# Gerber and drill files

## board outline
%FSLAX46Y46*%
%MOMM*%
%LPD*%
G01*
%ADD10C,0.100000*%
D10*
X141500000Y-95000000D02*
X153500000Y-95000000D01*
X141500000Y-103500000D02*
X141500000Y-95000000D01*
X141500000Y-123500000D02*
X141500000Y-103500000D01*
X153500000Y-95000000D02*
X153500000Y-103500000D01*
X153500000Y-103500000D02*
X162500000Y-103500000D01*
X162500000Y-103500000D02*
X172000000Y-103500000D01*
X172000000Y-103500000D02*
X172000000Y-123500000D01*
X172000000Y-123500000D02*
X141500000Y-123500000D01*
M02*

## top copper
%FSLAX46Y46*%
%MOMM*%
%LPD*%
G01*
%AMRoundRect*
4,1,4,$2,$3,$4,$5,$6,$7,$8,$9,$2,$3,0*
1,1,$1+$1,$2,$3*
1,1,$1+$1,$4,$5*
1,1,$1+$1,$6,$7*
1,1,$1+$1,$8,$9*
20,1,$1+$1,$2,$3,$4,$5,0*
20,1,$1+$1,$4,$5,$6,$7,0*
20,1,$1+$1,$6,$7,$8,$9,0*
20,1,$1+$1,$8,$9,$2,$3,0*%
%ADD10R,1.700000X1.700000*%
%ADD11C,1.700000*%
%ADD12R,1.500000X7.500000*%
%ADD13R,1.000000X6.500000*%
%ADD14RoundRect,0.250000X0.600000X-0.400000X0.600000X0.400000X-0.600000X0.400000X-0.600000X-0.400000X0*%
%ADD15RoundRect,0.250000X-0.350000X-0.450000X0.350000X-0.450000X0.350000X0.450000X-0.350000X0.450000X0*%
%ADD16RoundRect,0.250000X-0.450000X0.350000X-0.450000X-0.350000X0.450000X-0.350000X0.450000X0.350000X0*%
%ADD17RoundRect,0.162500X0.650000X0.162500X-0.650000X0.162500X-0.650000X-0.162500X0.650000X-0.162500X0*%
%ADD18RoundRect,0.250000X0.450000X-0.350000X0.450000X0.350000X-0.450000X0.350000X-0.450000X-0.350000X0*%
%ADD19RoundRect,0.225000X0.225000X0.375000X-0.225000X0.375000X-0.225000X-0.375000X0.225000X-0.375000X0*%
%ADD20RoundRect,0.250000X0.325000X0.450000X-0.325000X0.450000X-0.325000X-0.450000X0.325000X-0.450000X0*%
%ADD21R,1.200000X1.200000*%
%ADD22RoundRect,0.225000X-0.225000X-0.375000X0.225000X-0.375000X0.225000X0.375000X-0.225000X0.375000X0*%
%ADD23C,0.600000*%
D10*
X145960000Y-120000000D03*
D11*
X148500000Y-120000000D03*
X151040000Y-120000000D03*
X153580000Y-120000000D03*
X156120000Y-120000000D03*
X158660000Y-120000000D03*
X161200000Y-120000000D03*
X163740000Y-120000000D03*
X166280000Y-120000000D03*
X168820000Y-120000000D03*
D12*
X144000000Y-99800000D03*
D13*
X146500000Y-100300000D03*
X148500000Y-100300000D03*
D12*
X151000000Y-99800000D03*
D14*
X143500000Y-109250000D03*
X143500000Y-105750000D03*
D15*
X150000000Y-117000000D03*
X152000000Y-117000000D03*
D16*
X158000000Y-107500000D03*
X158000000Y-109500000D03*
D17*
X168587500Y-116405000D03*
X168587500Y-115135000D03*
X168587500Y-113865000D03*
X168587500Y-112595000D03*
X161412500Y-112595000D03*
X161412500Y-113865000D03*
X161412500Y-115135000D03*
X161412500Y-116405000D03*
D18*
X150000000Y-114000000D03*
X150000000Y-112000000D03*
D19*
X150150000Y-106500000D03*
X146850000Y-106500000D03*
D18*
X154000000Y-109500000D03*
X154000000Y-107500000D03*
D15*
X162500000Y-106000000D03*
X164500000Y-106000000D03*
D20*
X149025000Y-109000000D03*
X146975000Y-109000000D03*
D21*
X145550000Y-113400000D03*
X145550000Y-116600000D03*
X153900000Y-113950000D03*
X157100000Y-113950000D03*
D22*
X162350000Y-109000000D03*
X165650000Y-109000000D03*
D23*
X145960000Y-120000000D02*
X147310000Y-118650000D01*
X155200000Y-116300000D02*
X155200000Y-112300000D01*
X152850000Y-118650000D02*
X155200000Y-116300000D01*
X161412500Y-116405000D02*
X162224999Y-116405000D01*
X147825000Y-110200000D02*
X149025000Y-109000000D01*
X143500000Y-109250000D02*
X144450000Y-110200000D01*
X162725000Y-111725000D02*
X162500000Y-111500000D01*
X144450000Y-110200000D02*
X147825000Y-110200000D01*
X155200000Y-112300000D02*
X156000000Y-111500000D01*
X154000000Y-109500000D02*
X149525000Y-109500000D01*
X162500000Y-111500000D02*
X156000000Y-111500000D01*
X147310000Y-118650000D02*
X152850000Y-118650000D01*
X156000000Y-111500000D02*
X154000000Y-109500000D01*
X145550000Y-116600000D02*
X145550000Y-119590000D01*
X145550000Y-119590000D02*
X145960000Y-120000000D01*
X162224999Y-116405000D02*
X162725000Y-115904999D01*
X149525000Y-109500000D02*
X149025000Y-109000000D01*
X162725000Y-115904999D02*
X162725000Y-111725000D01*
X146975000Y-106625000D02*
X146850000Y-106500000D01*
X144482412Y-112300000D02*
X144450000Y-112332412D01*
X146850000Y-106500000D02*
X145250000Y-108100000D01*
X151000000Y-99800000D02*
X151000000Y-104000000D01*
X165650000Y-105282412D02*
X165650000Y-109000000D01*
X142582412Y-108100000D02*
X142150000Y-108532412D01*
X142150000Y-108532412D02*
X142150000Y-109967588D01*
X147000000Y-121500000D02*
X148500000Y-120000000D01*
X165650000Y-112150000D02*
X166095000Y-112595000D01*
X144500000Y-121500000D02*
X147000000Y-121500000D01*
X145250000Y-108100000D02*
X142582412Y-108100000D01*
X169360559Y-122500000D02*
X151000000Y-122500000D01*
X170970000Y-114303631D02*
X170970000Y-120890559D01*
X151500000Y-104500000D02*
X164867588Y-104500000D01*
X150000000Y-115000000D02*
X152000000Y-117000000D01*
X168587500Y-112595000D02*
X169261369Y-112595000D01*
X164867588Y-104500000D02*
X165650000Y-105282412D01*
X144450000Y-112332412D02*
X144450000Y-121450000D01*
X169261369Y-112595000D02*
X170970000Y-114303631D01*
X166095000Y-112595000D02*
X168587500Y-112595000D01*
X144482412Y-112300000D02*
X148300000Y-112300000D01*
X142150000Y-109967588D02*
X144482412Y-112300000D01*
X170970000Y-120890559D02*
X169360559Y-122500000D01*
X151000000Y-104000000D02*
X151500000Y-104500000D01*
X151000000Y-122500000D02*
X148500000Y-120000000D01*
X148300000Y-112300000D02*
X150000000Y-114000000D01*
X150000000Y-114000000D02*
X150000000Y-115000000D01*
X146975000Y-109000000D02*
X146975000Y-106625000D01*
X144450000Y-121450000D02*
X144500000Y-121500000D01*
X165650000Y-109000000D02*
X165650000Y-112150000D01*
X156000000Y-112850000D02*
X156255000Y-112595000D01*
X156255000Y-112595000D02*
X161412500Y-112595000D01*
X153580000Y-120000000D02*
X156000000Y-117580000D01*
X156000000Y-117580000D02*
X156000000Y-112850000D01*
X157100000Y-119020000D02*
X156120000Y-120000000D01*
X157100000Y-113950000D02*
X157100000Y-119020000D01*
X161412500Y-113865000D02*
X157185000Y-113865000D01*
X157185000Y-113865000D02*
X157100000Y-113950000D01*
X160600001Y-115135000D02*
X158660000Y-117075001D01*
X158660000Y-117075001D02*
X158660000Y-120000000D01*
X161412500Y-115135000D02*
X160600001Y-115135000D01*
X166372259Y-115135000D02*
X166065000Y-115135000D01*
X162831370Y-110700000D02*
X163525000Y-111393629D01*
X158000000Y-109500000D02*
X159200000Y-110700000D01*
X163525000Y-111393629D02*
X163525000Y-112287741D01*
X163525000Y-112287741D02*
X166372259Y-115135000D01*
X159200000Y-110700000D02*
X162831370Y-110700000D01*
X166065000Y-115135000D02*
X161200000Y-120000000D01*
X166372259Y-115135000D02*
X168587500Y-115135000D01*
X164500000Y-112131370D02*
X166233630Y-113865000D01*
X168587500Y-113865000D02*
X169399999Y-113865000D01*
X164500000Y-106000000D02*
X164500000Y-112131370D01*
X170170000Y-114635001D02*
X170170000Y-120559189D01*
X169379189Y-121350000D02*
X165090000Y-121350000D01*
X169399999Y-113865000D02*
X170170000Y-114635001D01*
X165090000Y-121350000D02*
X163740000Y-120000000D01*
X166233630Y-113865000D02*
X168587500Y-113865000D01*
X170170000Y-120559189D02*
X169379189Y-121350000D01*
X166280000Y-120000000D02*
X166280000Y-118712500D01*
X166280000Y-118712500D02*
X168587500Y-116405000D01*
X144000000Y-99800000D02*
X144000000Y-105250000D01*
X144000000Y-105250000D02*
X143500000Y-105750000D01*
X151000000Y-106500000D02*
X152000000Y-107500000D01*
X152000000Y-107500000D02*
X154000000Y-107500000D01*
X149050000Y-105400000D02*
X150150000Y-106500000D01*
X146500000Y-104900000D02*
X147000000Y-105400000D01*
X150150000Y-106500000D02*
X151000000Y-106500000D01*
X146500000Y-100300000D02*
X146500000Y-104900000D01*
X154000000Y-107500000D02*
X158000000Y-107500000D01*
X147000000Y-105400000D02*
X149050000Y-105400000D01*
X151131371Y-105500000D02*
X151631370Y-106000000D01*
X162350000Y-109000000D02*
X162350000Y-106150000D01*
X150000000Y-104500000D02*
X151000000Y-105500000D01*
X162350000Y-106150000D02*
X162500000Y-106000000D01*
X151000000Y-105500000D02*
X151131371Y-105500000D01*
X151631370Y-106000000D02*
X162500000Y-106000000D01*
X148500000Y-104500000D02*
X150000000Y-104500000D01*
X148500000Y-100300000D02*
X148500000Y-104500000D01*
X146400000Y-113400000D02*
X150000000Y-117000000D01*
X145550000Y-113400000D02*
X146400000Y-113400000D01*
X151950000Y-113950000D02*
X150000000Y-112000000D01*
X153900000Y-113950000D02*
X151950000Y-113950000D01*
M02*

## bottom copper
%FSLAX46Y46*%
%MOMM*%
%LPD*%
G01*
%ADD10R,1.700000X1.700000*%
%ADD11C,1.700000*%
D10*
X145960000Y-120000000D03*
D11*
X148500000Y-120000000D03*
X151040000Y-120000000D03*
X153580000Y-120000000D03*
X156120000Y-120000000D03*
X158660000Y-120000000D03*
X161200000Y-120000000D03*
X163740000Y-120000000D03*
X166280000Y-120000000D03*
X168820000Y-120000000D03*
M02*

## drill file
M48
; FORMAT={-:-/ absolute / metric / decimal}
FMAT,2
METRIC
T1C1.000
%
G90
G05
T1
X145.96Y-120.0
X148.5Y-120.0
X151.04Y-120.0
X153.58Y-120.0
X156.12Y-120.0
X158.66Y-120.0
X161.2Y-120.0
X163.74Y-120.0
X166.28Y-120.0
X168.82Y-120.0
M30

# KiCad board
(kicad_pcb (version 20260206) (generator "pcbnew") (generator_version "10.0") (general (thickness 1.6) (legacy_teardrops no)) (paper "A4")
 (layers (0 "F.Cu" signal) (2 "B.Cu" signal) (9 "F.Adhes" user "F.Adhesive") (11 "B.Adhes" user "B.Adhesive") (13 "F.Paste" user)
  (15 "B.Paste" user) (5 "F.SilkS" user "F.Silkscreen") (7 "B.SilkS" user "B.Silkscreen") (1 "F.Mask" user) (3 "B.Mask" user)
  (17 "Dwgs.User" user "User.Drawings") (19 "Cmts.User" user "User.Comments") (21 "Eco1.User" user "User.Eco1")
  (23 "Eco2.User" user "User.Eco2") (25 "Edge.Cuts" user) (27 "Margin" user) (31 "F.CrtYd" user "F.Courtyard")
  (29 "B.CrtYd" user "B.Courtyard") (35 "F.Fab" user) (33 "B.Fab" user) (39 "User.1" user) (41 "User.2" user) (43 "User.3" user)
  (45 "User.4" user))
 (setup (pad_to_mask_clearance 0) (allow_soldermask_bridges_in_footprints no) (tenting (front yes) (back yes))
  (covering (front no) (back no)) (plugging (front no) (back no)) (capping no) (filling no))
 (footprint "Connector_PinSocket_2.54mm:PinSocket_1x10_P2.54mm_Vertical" (layer "F.Cu") (at 145.96 120 90)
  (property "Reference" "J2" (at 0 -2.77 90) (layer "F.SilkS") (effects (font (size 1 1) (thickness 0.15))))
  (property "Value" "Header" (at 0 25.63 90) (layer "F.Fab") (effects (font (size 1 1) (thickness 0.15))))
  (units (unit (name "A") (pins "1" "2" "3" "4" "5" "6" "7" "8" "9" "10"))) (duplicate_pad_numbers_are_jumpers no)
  (pad "1" thru_hole rect (at 0 0 90) (size 1.7 1.7) (drill 1) (layers "*.Cu" "*.Mask") (remove_unused_layers no) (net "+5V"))
  (pad "2" thru_hole circle (at 0 2.54 90) (size 1.7 1.7) (drill 1) (layers "*.Cu" "*.Mask") (remove_unused_layers no) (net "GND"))
  (pad "3" thru_hole circle (at 0 5.08 90) (size 1.7 1.7) (drill 1) (layers "*.Cu" "*.Mask") (remove_unused_layers no)
   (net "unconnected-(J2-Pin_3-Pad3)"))
  (pad "4" thru_hole circle (at 0 7.62 90) (size 1.7 1.7) (drill 1) (layers "*.Cu" "*.Mask") (remove_unused_layers no)
   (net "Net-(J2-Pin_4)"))
  (pad "5" thru_hole circle (at 0 10.16 90) (size 1.7 1.7) (drill 1) (layers "*.Cu" "*.Mask") (remove_unused_layers no) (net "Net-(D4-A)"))
  (pad "6" thru_hole circle (at 0 12.7 90) (size 1.7 1.7) (drill 1) (layers "*.Cu" "*.Mask") (remove_unused_layers no)
   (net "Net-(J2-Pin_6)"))
  (pad "7" thru_hole circle (at 0 15.24 90) (size 1.7 1.7) (drill 1) (layers "*.Cu" "*.Mask") (remove_unused_layers no)
   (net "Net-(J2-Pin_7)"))
  (pad "8" thru_hole circle (at 0 17.78 90) (size 1.7 1.7) (drill 1) (layers "*.Cu" "*.Mask") (remove_unused_layers no)
   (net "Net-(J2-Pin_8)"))
  (pad "9" thru_hole circle (at 0 20.32 90) (size 1.7 1.7) (drill 1) (layers "*.Cu" "*.Mask") (remove_unused_layers no)
   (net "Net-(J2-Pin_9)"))
  (pad "10" thru_hole circle (at 0 22.86 90) (size 1.7 1.7) (drill 1) (layers "*.Cu" "*.Mask") (remove_unused_layers no)
   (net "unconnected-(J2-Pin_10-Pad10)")))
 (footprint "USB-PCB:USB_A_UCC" (layer "F.Cu") (at 147.5 100 -90)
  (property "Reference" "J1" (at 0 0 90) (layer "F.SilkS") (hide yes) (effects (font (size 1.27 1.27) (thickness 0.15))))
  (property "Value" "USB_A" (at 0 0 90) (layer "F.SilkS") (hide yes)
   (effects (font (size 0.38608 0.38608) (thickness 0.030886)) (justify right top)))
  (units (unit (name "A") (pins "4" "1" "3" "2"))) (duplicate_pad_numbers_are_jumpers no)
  (pad "1" smd rect (at -0.2 3.5 270) (size 7.5 1.5) (layers "F.Cu" "F.Mask" "F.Paste") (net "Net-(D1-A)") (solder_mask_margin 0.1016))
  (pad "2" smd rect (at 0.3 1 270) (size 6.5 1) (layers "F.Cu" "F.Mask" "F.Paste") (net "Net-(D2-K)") (solder_mask_margin 0.1016))
  (pad "3" smd rect (at 0.3 -1 270) (size 6.5 1) (layers "F.Cu" "F.Mask" "F.Paste") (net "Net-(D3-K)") (solder_mask_margin 0.1016))
  (pad "4" smd rect (at -0.2 -3.5 270) (size 7.5 1.5) (layers "F.Cu" "F.Mask" "F.Paste") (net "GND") (solder_mask_margin 0.1016)))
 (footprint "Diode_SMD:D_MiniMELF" (layer "F.Cu") (at 143.5 107.5 90)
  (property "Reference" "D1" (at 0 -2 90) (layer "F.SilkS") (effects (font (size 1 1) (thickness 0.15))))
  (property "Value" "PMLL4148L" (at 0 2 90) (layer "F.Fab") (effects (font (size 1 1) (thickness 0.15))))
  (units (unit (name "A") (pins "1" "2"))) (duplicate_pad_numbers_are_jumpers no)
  (pad "1" smd roundrect (at -1.75 0 90) (size 1.3 1.7) (layers "F.Cu" "F.Mask" "F.Paste") (roundrect_rratio 0.1923076923) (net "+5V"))
  (pad "2" smd roundrect (at 1.75 0 90) (size 1.3 1.7) (layers "F.Cu" "F.Mask" "F.Paste") (roundrect_rratio 0.1923076923) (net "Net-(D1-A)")))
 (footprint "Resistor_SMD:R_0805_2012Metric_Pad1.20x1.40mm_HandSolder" (layer "F.Cu") (at 151 117)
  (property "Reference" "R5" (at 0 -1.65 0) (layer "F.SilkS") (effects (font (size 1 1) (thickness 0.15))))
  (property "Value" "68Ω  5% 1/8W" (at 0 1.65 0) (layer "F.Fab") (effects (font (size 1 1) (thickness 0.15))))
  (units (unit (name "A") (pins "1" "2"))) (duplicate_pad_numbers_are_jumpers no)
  (pad "1" smd roundrect (at -1 0) (size 1.2 1.4) (layers "F.Cu" "F.Mask" "F.Paste") (roundrect_rratio 0.208333) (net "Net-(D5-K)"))
  (pad "2" smd roundrect (at 1 0) (size 1.2 1.4) (layers "F.Cu" "F.Mask" "F.Paste") (roundrect_rratio 0.208333) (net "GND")))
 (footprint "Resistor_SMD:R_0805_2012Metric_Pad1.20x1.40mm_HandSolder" (layer "F.Cu") (at 158 108.5 -90)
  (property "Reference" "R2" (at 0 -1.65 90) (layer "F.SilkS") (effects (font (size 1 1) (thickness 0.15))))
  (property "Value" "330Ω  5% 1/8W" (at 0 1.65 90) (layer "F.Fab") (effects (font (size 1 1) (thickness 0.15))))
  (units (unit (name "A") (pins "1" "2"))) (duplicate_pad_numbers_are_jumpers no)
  (pad "1" smd roundrect (at -1 0 270) (size 1.2 1.4) (layers "F.Cu" "F.Mask" "F.Paste") (roundrect_rratio 0.208333) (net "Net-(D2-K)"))
  (pad "2" smd roundrect (at 1 0 270) (size 1.2 1.4) (layers "F.Cu" "F.Mask" "F.Paste") (roundrect_rratio 0.208333) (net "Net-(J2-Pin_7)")))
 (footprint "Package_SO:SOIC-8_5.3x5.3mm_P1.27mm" (layer "F.Cu") (at 165 114.5 180)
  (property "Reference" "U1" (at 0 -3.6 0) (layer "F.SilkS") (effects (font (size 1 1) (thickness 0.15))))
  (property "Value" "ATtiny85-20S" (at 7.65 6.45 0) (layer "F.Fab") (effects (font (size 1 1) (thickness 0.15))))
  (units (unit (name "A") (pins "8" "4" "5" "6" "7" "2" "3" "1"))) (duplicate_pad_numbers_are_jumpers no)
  (pad "1" smd roundrect (at -3.5875 -1.905 180) (size 1.625 0.65) (layers "F.Cu" "F.Mask" "F.Paste") (roundrect_rratio 0.25)
   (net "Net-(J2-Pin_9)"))
  (pad "2" smd roundrect (at -3.5875 -0.635 180) (size 1.625 0.65) (layers "F.Cu" "F.Mask" "F.Paste") (roundrect_rratio 0.25)
   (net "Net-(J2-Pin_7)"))
  (pad "3" smd roundrect (at -3.5875 0.635 180) (size 1.625 0.65) (layers "F.Cu" "F.Mask" "F.Paste") (roundrect_rratio 0.25)
   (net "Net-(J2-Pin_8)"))
  (pad "4" smd roundrect (at -3.5875 1.905 180) (size 1.625 0.65) (layers "F.Cu" "F.Mask" "F.Paste") (roundrect_rratio 0.25) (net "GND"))
  (pad "5" smd roundrect (at 3.5875 1.905 180) (size 1.625 0.65) (layers "F.Cu" "F.Mask" "F.Paste") (roundrect_rratio 0.25)
   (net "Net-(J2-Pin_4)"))
  (pad "6" smd roundrect (at 3.5875 0.635 180) (size 1.625 0.65) (layers "F.Cu" "F.Mask" "F.Paste") (roundrect_rratio 0.25)
   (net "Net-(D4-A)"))
  (pad "7" smd roundrect (at 3.5875 -0.635 180) (size 1.625 0.65) (layers "F.Cu" "F.Mask" "F.Paste") (roundrect_rratio 0.25)
   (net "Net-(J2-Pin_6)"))
  (pad "8" smd roundrect (at 3.5875 -1.905 180) (size 1.625 0.65) (layers "F.Cu" "F.Mask" "F.Paste") (roundrect_rratio 0.25) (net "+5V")))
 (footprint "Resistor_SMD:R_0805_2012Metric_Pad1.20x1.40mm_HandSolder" (layer "F.Cu") (at 150 113 90)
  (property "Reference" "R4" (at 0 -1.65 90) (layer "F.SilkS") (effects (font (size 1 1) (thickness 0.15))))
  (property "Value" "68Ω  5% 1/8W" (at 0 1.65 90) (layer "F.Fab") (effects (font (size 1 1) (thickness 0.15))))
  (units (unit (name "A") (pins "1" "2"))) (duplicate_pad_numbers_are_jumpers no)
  (pad "1" smd roundrect (at -1 0 90) (size 1.2 1.4) (layers "F.Cu" "F.Mask" "F.Paste") (roundrect_rratio 0.208333) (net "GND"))
  (pad "2" smd roundrect (at 1 0 90) (size 1.2 1.4) (layers "F.Cu" "F.Mask" "F.Paste") (roundrect_rratio 0.208333) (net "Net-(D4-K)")))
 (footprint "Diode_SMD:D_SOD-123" (layer "F.Cu") (at 148.5 106.5 180)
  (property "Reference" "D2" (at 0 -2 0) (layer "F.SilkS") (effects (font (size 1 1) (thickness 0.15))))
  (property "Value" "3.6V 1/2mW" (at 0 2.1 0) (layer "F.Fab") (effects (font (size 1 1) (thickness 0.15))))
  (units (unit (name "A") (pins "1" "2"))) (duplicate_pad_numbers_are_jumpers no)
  (pad "1" smd roundrect (at -1.65 0 180) (size 0.9 1.2) (layers "F.Cu" "F.Mask" "F.Paste") (roundrect_rratio 0.25) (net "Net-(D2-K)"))
  (pad "2" smd roundrect (at 1.65 0 180) (size 0.9 1.2) (layers "F.Cu" "F.Mask" "F.Paste") (roundrect_rratio 0.25) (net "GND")))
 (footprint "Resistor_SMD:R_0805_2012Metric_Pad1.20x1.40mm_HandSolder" (layer "F.Cu") (at 154 108.5 90)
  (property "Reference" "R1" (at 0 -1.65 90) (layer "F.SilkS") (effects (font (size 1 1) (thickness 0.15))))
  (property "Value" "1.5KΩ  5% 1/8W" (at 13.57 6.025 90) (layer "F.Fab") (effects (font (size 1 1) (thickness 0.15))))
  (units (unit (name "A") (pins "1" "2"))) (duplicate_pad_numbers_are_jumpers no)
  (pad "1" smd roundrect (at -1 0 90) (size 1.2 1.4) (layers "F.Cu" "F.Mask" "F.Paste") (roundrect_rratio 0.208333) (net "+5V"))
  (pad "2" smd roundrect (at 1 0 90) (size 1.2 1.4) (layers "F.Cu" "F.Mask" "F.Paste") (roundrect_rratio 0.208333) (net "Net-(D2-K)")))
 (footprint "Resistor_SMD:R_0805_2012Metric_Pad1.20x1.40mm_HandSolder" (layer "F.Cu") (at 163.5 106)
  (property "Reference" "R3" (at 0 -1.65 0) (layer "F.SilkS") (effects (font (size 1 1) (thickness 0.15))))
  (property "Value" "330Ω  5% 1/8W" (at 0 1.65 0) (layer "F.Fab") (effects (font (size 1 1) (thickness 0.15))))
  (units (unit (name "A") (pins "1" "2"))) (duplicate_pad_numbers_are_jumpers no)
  (pad "1" smd roundrect (at -1 0) (size 1.2 1.4) (layers "F.Cu" "F.Mask" "F.Paste") (roundrect_rratio 0.208333) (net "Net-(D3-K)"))
  (pad "2" smd roundrect (at 1 0) (size 1.2 1.4) (layers "F.Cu" "F.Mask" "F.Paste") (roundrect_rratio 0.208333) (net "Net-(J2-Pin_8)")))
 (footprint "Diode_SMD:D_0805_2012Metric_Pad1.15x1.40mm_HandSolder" (layer "F.Cu") (at 148 109 180)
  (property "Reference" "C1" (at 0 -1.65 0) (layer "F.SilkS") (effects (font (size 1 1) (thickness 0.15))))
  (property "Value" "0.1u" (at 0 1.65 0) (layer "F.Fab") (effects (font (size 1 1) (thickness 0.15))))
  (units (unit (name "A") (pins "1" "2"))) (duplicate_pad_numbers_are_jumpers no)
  (pad "1" smd roundrect (at -1.025 0 180) (size 1.15 1.4) (layers "F.Cu" "F.Mask" "F.Paste") (roundrect_rratio 0.217391) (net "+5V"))
  (pad "2" smd roundrect (at 1.025 0 180) (size 1.15 1.4) (layers "F.Cu" "F.Mask" "F.Paste") (roundrect_rratio 0.217391) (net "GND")))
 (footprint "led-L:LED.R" (layer "F.Cu") (at 146 115.5 -90)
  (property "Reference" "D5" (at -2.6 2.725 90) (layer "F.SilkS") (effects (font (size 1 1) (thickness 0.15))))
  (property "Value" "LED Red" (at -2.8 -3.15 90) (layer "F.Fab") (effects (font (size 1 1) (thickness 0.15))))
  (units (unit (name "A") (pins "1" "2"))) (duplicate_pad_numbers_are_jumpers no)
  (pad "1" smd rect (at -2.1 0.45 270) (size 1.2 1.2) (layers "F.Cu" "F.Mask" "F.Paste") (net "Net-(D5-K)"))
  (pad "2" smd rect (at 1.1 0.45 270) (size 1.2 1.2) (layers "F.Cu" "F.Mask" "F.Paste") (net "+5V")))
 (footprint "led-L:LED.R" (layer "F.Cu") (at 156 113.5)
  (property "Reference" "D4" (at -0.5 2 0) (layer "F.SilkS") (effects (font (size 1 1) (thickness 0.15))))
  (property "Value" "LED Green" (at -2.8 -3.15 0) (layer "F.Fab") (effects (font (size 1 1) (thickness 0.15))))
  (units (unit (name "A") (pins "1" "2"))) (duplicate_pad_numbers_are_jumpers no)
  (pad "1" smd rect (at -2.1 0.45) (size 1.2 1.2) (layers "F.Cu" "F.Mask" "F.Paste") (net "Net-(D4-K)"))
  (pad "2" smd rect (at 1.1 0.45) (size 1.2 1.2) (layers "F.Cu" "F.Mask" "F.Paste") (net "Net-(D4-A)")))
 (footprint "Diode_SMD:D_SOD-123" (layer "F.Cu") (at 164 109)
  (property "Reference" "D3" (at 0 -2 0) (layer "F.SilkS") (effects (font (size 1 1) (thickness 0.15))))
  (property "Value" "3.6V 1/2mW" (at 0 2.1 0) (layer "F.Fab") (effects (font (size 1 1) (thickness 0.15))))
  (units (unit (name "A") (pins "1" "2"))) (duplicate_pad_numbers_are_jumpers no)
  (pad "1" smd roundrect (at -1.65 0) (size 0.9 1.2) (layers "F.Cu" "F.Mask" "F.Paste") (roundrect_rratio 0.25) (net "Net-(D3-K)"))
  (pad "2" smd roundrect (at 1.65 0) (size 0.9 1.2) (layers "F.Cu" "F.Mask" "F.Paste") (roundrect_rratio 0.25) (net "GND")))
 (gr_line (start 141.5 95) (end 153.5 95) (stroke (width 0.1) (type default)) (layer "Edge.Cuts"))
 (gr_line (start 141.5 103.5) (end 141.5 95) (stroke (width 0.1) (type default)) (layer "Edge.Cuts"))
 (gr_line (start 141.5 123.5) (end 141.5 103.5) (stroke (width 0.1) (type default)) (layer "Edge.Cuts"))
 (gr_line (start 153.5 95) (end 153.5 103.5) (stroke (width 0.1) (type default)) (layer "Edge.Cuts"))
 (gr_line (start 153.5 103.5) (end 162.5 103.5) (stroke (width 0.1) (type default)) (layer "Edge.Cuts"))
 (gr_line (start 162.5 103.5) (end 172 103.5) (stroke (width 0.1) (type default)) (layer "Edge.Cuts"))
 (gr_line (start 172 103.5) (end 172 123.5) (stroke (width 0.1) (type default)) (layer "Edge.Cuts"))
 (gr_line (start 172 123.5) (end 141.5 123.5) (stroke (width 0.1) (type default)) (layer "Edge.Cuts"))
 (segment (start 145.96 120) (end 147.31 118.65) (width 0.6) (layer "F.Cu") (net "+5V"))
 (segment (start 155.2 116.3) (end 155.2 112.3) (width 0.6) (layer "F.Cu") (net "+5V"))
 (segment (start 152.85 118.65) (end 155.2 116.3) (width 0.6) (layer "F.Cu") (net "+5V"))
 (segment (start 161.4125 116.405) (end 162.224999 116.405) (width 0.6) (layer "F.Cu") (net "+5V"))
 (segment (start 147.825 110.2) (end 149.025 109) (width 0.6) (layer "F.Cu") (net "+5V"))
 (segment (start 143.5 109.25) (end 144.45 110.2) (width 0.6) (layer "F.Cu") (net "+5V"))
 (segment (start 162.725 111.725) (end 162.5 111.5) (width 0.6) (layer "F.Cu") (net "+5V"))
 (segment (start 144.45 110.2) (end 147.825 110.2) (width 0.6) (layer "F.Cu") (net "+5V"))
 (segment (start 155.2 112.3) (end 156 111.5) (width 0.6) (layer "F.Cu") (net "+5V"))
 (segment (start 154 109.5) (end 149.525 109.5) (width 0.6) (layer "F.Cu") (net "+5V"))
 (segment (start 162.5 111.5) (end 156 111.5) (width 0.6) (layer "F.Cu") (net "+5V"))
 (segment (start 147.31 118.65) (end 152.85 118.65) (width 0.6) (layer "F.Cu") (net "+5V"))
 (segment (start 156 111.5) (end 154 109.5) (width 0.6) (layer "F.Cu") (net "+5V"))
 (segment (start 145.55 116.6) (end 145.55 119.59) (width 0.6) (layer "F.Cu") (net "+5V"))
 (segment (start 145.55 119.59) (end 145.96 120) (width 0.6) (layer "F.Cu") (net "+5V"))
 (segment (start 162.224999 116.405) (end 162.725 115.904999) (width 0.6) (layer "F.Cu") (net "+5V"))
 (segment (start 149.525 109.5) (end 149.025 109) (width 0.6) (layer "F.Cu") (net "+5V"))
 (segment (start 162.725 115.904999) (end 162.725 111.725) (width 0.6) (layer "F.Cu") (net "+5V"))
 (segment (start 146.975 106.625) (end 146.85 106.5) (width 0.6) (layer "F.Cu") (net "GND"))
 (segment (start 144.482412 112.3) (end 144.45 112.332412) (width 0.6) (layer "F.Cu") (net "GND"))
 (segment (start 146.85 106.5) (end 145.25 108.1) (width 0.6) (layer "F.Cu") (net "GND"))
 (segment (start 151 99.8) (end 151 104) (width 0.6) (layer "F.Cu") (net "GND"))
 (segment (start 165.65 105.282412) (end 165.65 109) (width 0.6) (layer "F.Cu") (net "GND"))
 (segment (start 142.582412 108.1) (end 142.15 108.532412) (width 0.6) (layer "F.Cu") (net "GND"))
 (segment (start 142.15 108.532412) (end 142.15 109.967588) (width 0.6) (layer "F.Cu") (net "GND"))
 (segment (start 147 121.5) (end 148.5 120) (width 0.6) (layer "F.Cu") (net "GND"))
 (segment (start 165.65 112.15) (end 166.095 112.595) (width 0.6) (layer "F.Cu") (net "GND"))
 (segment (start 144.5 121.5) (end 147 121.5) (width 0.6) (layer "F.Cu") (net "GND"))
 (segment (start 145.25 108.1) (end 142.582412 108.1) (width 0.6) (layer "F.Cu") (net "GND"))
 (segment (start 169.360559 122.5) (end 151 122.5) (width 0.6) (layer "F.Cu") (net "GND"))
 (segment (start 170.97 114.303631) (end 170.97 120.890559) (width 0.6) (layer "F.Cu") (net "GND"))
 (segment (start 151.5 104.5) (end 164.867588 104.5) (width 0.6) (layer "F.Cu") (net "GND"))
 (segment (start 150 115) (end 152 117) (width 0.6) (layer "F.Cu") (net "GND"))
 (segment (start 168.5875 112.595) (end 169.261369 112.595) (width 0.6) (layer "F.Cu") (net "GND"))
 (segment (start 164.867588 104.5) (end 165.65 105.282412) (width 0.6) (layer "F.Cu") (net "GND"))
 (segment (start 144.45 112.332412) (end 144.45 121.45) (width 0.6) (layer "F.Cu") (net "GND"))
 (segment (start 169.261369 112.595) (end 170.97 114.303631) (width 0.6) (layer "F.Cu") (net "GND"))
 (segment (start 166.095 112.595) (end 168.5875 112.595) (width 0.6) (layer "F.Cu") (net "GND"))
 (segment (start 144.482412 112.3) (end 148.3 112.3) (width 0.6) (layer "F.Cu") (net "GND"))
 (segment (start 142.15 109.967588) (end 144.482412 112.3) (width 0.6) (layer "F.Cu") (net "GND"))
 (segment (start 170.97 120.890559) (end 169.360559 122.5) (width 0.6) (layer "F.Cu") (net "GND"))
 (segment (start 151 104) (end 151.5 104.5) (width 0.6) (layer "F.Cu") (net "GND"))
 (segment (start 151 122.5) (end 148.5 120) (width 0.6) (layer "F.Cu") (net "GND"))
 (segment (start 148.3 112.3) (end 150 114) (width 0.6) (layer "F.Cu") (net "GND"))
 (segment (start 150 114) (end 150 115) (width 0.6) (layer "F.Cu") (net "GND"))
 (segment (start 146.975 109) (end 146.975 106.625) (width 0.6) (layer "F.Cu") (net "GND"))
 (segment (start 144.45 121.45) (end 144.5 121.5) (width 0.6) (layer "F.Cu") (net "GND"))
 (segment (start 165.65 109) (end 165.65 112.15) (width 0.6) (layer "F.Cu") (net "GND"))
 (segment (start 156 112.85) (end 156.255 112.595) (width 0.6) (layer "F.Cu") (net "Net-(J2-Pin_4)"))
 (segment (start 156.255 112.595) (end 161.4125 112.595) (width 0.6) (layer "F.Cu") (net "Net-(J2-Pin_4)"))
 (segment (start 153.58 120) (end 156 117.58) (width 0.6) (layer "F.Cu") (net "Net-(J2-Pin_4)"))
 (segment (start 156 117.58) (end 156 112.85) (width 0.6) (layer "F.Cu") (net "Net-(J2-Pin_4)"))
 (segment (start 157.1 119.02) (end 156.12 120) (width 0.6) (layer "F.Cu") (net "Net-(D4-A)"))
 (segment (start 157.1 113.95) (end 157.1 119.02) (width 0.6) (layer "F.Cu") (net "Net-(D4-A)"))
 (segment (start 161.4125 113.865) (end 157.185 113.865) (width 0.6) (layer "F.Cu") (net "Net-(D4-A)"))
 (segment (start 157.185 113.865) (end 157.1 113.95) (width 0.6) (layer "F.Cu") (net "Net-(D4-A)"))
 (segment (start 160.600001 115.135) (end 158.66 117.075001) (width 0.6) (layer "F.Cu") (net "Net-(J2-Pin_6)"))
 (segment (start 158.66 117.075001) (end 158.66 120) (width 0.6) (layer "F.Cu") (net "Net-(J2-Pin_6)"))
 (segment (start 161.4125 115.135) (end 160.600001 115.135) (width 0.6) (layer "F.Cu") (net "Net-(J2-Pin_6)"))
 (segment (start 166.372259 115.135) (end 166.065 115.135) (width 0.6) (layer "F.Cu") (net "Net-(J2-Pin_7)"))
 (segment (start 162.83137 110.7) (end 163.525 111.393629) (width 0.6) (layer "F.Cu") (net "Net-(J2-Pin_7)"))
 (segment (start 158 109.5) (end 159.2 110.7) (width 0.6) (layer "F.Cu") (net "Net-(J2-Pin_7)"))
 (segment (start 163.525 111.393629) (end 163.525 112.287741) (width 0.6) (layer "F.Cu") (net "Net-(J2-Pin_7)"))
 (segment (start 163.525 112.287741) (end 166.372259 115.135) (width 0.6) (layer "F.Cu") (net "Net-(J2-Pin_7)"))
 (segment (start 159.2 110.7) (end 162.83137 110.7) (width 0.6) (layer "F.Cu") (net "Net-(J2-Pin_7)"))
 (segment (start 166.065 115.135) (end 161.2 120) (width 0.6) (layer "F.Cu") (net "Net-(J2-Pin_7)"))
 (segment (start 166.372259 115.135) (end 168.5875 115.135) (width 0.6) (layer "F.Cu") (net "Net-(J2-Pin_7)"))
 (segment (start 164.5 112.13137) (end 166.23363 113.865) (width 0.6) (layer "F.Cu") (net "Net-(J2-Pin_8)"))
 (segment (start 168.5875 113.865) (end 169.399999 113.865) (width 0.6) (layer "F.Cu") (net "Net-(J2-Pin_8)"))
 (segment (start 164.5 106) (end 164.5 112.13137) (width 0.6) (layer "F.Cu") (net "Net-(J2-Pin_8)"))
 (segment (start 170.17 114.635001) (end 170.17 120.559189) (width 0.6) (layer "F.Cu") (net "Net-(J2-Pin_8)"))
 (segment (start 169.379189 121.35) (end 165.09 121.35) (width 0.6) (layer "F.Cu") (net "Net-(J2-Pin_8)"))
 (segment (start 169.399999 113.865) (end 170.17 114.635001) (width 0.6) (layer "F.Cu") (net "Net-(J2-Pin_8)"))
 (segment (start 165.09 121.35) (end 163.74 120) (width 0.6) (layer "F.Cu") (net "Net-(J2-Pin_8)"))
 (segment (start 166.23363 113.865) (end 168.5875 113.865) (width 0.6) (layer "F.Cu") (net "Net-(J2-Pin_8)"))
 (segment (start 170.17 120.559189) (end 169.379189 121.35) (width 0.6) (layer "F.Cu") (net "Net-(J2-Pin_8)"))
 (segment (start 166.28 120) (end 166.28 118.7125) (width 0.6) (layer "F.Cu") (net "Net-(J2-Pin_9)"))
 (segment (start 166.28 118.7125) (end 168.5875 116.405) (width 0.6) (layer "F.Cu") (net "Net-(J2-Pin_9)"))
 (segment (start 144 99.8) (end 144 105.25) (width 0.6) (layer "F.Cu") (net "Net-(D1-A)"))
 (segment (start 144 105.25) (end 143.5 105.75) (width 0.6) (layer "F.Cu") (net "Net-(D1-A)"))
 (segment (start 151 106.5) (end 152 107.5) (width 0.6) (layer "F.Cu") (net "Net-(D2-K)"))
 (segment (start 152 107.5) (end 154 107.5) (width 0.6) (layer "F.Cu") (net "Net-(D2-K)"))
 (segment (start 149.05 105.4) (end 150.15 106.5) (width 0.6) (layer "F.Cu") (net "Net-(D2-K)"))
 (segment (start 146.5 104.9) (end 147 105.4) (width 0.6) (layer "F.Cu") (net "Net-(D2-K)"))
 (segment (start 150.15 106.5) (end 151 106.5) (width 0.6) (layer "F.Cu") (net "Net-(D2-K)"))
 (segment (start 146.5 100.3) (end 146.5 104.9) (width 0.6) (layer "F.Cu") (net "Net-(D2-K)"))
 (segment (start 154 107.5) (end 158 107.5) (width 0.6) (layer "F.Cu") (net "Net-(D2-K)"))
 (segment (start 147 105.4) (end 149.05 105.4) (width 0.6) (layer "F.Cu") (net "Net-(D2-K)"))
 (segment (start 151.131371 105.5) (end 151.63137 106) (width 0.6) (layer "F.Cu") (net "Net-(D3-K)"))
 (segment (start 162.35 109) (end 162.35 106.15) (width 0.6) (layer "F.Cu") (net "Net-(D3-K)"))
 (segment (start 150 104.5) (end 151 105.5) (width 0.6) (layer "F.Cu") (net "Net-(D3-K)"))
 (segment (start 162.35 106.15) (end 162.5 106) (width 0.6) (layer "F.Cu") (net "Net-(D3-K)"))
 (segment (start 151 105.5) (end 151.131371 105.5) (width 0.6) (layer "F.Cu") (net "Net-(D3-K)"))
 (segment (start 151.63137 106) (end 162.5 106) (width 0.6) (layer "F.Cu") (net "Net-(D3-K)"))
 (segment (start 148.5 104.5) (end 150 104.5) (width 0.6) (layer "F.Cu") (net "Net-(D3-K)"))
 (segment (start 148.5 100.3) (end 148.5 104.5) (width 0.6) (layer "F.Cu") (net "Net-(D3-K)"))
 (segment (start 146.4 113.4) (end 150 117) (width 0.6) (layer "F.Cu") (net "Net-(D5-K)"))
 (segment (start 145.55 113.4) (end 146.4 113.4) (width 0.6) (layer "F.Cu") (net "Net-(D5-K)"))
 (segment (start 151.95 113.95) (end 150 112) (width 0.6) (layer "F.Cu") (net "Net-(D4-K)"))
 (segment (start 153.9 113.95) (end 151.95 113.95) (width 0.6) (layer "F.Cu") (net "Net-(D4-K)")))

